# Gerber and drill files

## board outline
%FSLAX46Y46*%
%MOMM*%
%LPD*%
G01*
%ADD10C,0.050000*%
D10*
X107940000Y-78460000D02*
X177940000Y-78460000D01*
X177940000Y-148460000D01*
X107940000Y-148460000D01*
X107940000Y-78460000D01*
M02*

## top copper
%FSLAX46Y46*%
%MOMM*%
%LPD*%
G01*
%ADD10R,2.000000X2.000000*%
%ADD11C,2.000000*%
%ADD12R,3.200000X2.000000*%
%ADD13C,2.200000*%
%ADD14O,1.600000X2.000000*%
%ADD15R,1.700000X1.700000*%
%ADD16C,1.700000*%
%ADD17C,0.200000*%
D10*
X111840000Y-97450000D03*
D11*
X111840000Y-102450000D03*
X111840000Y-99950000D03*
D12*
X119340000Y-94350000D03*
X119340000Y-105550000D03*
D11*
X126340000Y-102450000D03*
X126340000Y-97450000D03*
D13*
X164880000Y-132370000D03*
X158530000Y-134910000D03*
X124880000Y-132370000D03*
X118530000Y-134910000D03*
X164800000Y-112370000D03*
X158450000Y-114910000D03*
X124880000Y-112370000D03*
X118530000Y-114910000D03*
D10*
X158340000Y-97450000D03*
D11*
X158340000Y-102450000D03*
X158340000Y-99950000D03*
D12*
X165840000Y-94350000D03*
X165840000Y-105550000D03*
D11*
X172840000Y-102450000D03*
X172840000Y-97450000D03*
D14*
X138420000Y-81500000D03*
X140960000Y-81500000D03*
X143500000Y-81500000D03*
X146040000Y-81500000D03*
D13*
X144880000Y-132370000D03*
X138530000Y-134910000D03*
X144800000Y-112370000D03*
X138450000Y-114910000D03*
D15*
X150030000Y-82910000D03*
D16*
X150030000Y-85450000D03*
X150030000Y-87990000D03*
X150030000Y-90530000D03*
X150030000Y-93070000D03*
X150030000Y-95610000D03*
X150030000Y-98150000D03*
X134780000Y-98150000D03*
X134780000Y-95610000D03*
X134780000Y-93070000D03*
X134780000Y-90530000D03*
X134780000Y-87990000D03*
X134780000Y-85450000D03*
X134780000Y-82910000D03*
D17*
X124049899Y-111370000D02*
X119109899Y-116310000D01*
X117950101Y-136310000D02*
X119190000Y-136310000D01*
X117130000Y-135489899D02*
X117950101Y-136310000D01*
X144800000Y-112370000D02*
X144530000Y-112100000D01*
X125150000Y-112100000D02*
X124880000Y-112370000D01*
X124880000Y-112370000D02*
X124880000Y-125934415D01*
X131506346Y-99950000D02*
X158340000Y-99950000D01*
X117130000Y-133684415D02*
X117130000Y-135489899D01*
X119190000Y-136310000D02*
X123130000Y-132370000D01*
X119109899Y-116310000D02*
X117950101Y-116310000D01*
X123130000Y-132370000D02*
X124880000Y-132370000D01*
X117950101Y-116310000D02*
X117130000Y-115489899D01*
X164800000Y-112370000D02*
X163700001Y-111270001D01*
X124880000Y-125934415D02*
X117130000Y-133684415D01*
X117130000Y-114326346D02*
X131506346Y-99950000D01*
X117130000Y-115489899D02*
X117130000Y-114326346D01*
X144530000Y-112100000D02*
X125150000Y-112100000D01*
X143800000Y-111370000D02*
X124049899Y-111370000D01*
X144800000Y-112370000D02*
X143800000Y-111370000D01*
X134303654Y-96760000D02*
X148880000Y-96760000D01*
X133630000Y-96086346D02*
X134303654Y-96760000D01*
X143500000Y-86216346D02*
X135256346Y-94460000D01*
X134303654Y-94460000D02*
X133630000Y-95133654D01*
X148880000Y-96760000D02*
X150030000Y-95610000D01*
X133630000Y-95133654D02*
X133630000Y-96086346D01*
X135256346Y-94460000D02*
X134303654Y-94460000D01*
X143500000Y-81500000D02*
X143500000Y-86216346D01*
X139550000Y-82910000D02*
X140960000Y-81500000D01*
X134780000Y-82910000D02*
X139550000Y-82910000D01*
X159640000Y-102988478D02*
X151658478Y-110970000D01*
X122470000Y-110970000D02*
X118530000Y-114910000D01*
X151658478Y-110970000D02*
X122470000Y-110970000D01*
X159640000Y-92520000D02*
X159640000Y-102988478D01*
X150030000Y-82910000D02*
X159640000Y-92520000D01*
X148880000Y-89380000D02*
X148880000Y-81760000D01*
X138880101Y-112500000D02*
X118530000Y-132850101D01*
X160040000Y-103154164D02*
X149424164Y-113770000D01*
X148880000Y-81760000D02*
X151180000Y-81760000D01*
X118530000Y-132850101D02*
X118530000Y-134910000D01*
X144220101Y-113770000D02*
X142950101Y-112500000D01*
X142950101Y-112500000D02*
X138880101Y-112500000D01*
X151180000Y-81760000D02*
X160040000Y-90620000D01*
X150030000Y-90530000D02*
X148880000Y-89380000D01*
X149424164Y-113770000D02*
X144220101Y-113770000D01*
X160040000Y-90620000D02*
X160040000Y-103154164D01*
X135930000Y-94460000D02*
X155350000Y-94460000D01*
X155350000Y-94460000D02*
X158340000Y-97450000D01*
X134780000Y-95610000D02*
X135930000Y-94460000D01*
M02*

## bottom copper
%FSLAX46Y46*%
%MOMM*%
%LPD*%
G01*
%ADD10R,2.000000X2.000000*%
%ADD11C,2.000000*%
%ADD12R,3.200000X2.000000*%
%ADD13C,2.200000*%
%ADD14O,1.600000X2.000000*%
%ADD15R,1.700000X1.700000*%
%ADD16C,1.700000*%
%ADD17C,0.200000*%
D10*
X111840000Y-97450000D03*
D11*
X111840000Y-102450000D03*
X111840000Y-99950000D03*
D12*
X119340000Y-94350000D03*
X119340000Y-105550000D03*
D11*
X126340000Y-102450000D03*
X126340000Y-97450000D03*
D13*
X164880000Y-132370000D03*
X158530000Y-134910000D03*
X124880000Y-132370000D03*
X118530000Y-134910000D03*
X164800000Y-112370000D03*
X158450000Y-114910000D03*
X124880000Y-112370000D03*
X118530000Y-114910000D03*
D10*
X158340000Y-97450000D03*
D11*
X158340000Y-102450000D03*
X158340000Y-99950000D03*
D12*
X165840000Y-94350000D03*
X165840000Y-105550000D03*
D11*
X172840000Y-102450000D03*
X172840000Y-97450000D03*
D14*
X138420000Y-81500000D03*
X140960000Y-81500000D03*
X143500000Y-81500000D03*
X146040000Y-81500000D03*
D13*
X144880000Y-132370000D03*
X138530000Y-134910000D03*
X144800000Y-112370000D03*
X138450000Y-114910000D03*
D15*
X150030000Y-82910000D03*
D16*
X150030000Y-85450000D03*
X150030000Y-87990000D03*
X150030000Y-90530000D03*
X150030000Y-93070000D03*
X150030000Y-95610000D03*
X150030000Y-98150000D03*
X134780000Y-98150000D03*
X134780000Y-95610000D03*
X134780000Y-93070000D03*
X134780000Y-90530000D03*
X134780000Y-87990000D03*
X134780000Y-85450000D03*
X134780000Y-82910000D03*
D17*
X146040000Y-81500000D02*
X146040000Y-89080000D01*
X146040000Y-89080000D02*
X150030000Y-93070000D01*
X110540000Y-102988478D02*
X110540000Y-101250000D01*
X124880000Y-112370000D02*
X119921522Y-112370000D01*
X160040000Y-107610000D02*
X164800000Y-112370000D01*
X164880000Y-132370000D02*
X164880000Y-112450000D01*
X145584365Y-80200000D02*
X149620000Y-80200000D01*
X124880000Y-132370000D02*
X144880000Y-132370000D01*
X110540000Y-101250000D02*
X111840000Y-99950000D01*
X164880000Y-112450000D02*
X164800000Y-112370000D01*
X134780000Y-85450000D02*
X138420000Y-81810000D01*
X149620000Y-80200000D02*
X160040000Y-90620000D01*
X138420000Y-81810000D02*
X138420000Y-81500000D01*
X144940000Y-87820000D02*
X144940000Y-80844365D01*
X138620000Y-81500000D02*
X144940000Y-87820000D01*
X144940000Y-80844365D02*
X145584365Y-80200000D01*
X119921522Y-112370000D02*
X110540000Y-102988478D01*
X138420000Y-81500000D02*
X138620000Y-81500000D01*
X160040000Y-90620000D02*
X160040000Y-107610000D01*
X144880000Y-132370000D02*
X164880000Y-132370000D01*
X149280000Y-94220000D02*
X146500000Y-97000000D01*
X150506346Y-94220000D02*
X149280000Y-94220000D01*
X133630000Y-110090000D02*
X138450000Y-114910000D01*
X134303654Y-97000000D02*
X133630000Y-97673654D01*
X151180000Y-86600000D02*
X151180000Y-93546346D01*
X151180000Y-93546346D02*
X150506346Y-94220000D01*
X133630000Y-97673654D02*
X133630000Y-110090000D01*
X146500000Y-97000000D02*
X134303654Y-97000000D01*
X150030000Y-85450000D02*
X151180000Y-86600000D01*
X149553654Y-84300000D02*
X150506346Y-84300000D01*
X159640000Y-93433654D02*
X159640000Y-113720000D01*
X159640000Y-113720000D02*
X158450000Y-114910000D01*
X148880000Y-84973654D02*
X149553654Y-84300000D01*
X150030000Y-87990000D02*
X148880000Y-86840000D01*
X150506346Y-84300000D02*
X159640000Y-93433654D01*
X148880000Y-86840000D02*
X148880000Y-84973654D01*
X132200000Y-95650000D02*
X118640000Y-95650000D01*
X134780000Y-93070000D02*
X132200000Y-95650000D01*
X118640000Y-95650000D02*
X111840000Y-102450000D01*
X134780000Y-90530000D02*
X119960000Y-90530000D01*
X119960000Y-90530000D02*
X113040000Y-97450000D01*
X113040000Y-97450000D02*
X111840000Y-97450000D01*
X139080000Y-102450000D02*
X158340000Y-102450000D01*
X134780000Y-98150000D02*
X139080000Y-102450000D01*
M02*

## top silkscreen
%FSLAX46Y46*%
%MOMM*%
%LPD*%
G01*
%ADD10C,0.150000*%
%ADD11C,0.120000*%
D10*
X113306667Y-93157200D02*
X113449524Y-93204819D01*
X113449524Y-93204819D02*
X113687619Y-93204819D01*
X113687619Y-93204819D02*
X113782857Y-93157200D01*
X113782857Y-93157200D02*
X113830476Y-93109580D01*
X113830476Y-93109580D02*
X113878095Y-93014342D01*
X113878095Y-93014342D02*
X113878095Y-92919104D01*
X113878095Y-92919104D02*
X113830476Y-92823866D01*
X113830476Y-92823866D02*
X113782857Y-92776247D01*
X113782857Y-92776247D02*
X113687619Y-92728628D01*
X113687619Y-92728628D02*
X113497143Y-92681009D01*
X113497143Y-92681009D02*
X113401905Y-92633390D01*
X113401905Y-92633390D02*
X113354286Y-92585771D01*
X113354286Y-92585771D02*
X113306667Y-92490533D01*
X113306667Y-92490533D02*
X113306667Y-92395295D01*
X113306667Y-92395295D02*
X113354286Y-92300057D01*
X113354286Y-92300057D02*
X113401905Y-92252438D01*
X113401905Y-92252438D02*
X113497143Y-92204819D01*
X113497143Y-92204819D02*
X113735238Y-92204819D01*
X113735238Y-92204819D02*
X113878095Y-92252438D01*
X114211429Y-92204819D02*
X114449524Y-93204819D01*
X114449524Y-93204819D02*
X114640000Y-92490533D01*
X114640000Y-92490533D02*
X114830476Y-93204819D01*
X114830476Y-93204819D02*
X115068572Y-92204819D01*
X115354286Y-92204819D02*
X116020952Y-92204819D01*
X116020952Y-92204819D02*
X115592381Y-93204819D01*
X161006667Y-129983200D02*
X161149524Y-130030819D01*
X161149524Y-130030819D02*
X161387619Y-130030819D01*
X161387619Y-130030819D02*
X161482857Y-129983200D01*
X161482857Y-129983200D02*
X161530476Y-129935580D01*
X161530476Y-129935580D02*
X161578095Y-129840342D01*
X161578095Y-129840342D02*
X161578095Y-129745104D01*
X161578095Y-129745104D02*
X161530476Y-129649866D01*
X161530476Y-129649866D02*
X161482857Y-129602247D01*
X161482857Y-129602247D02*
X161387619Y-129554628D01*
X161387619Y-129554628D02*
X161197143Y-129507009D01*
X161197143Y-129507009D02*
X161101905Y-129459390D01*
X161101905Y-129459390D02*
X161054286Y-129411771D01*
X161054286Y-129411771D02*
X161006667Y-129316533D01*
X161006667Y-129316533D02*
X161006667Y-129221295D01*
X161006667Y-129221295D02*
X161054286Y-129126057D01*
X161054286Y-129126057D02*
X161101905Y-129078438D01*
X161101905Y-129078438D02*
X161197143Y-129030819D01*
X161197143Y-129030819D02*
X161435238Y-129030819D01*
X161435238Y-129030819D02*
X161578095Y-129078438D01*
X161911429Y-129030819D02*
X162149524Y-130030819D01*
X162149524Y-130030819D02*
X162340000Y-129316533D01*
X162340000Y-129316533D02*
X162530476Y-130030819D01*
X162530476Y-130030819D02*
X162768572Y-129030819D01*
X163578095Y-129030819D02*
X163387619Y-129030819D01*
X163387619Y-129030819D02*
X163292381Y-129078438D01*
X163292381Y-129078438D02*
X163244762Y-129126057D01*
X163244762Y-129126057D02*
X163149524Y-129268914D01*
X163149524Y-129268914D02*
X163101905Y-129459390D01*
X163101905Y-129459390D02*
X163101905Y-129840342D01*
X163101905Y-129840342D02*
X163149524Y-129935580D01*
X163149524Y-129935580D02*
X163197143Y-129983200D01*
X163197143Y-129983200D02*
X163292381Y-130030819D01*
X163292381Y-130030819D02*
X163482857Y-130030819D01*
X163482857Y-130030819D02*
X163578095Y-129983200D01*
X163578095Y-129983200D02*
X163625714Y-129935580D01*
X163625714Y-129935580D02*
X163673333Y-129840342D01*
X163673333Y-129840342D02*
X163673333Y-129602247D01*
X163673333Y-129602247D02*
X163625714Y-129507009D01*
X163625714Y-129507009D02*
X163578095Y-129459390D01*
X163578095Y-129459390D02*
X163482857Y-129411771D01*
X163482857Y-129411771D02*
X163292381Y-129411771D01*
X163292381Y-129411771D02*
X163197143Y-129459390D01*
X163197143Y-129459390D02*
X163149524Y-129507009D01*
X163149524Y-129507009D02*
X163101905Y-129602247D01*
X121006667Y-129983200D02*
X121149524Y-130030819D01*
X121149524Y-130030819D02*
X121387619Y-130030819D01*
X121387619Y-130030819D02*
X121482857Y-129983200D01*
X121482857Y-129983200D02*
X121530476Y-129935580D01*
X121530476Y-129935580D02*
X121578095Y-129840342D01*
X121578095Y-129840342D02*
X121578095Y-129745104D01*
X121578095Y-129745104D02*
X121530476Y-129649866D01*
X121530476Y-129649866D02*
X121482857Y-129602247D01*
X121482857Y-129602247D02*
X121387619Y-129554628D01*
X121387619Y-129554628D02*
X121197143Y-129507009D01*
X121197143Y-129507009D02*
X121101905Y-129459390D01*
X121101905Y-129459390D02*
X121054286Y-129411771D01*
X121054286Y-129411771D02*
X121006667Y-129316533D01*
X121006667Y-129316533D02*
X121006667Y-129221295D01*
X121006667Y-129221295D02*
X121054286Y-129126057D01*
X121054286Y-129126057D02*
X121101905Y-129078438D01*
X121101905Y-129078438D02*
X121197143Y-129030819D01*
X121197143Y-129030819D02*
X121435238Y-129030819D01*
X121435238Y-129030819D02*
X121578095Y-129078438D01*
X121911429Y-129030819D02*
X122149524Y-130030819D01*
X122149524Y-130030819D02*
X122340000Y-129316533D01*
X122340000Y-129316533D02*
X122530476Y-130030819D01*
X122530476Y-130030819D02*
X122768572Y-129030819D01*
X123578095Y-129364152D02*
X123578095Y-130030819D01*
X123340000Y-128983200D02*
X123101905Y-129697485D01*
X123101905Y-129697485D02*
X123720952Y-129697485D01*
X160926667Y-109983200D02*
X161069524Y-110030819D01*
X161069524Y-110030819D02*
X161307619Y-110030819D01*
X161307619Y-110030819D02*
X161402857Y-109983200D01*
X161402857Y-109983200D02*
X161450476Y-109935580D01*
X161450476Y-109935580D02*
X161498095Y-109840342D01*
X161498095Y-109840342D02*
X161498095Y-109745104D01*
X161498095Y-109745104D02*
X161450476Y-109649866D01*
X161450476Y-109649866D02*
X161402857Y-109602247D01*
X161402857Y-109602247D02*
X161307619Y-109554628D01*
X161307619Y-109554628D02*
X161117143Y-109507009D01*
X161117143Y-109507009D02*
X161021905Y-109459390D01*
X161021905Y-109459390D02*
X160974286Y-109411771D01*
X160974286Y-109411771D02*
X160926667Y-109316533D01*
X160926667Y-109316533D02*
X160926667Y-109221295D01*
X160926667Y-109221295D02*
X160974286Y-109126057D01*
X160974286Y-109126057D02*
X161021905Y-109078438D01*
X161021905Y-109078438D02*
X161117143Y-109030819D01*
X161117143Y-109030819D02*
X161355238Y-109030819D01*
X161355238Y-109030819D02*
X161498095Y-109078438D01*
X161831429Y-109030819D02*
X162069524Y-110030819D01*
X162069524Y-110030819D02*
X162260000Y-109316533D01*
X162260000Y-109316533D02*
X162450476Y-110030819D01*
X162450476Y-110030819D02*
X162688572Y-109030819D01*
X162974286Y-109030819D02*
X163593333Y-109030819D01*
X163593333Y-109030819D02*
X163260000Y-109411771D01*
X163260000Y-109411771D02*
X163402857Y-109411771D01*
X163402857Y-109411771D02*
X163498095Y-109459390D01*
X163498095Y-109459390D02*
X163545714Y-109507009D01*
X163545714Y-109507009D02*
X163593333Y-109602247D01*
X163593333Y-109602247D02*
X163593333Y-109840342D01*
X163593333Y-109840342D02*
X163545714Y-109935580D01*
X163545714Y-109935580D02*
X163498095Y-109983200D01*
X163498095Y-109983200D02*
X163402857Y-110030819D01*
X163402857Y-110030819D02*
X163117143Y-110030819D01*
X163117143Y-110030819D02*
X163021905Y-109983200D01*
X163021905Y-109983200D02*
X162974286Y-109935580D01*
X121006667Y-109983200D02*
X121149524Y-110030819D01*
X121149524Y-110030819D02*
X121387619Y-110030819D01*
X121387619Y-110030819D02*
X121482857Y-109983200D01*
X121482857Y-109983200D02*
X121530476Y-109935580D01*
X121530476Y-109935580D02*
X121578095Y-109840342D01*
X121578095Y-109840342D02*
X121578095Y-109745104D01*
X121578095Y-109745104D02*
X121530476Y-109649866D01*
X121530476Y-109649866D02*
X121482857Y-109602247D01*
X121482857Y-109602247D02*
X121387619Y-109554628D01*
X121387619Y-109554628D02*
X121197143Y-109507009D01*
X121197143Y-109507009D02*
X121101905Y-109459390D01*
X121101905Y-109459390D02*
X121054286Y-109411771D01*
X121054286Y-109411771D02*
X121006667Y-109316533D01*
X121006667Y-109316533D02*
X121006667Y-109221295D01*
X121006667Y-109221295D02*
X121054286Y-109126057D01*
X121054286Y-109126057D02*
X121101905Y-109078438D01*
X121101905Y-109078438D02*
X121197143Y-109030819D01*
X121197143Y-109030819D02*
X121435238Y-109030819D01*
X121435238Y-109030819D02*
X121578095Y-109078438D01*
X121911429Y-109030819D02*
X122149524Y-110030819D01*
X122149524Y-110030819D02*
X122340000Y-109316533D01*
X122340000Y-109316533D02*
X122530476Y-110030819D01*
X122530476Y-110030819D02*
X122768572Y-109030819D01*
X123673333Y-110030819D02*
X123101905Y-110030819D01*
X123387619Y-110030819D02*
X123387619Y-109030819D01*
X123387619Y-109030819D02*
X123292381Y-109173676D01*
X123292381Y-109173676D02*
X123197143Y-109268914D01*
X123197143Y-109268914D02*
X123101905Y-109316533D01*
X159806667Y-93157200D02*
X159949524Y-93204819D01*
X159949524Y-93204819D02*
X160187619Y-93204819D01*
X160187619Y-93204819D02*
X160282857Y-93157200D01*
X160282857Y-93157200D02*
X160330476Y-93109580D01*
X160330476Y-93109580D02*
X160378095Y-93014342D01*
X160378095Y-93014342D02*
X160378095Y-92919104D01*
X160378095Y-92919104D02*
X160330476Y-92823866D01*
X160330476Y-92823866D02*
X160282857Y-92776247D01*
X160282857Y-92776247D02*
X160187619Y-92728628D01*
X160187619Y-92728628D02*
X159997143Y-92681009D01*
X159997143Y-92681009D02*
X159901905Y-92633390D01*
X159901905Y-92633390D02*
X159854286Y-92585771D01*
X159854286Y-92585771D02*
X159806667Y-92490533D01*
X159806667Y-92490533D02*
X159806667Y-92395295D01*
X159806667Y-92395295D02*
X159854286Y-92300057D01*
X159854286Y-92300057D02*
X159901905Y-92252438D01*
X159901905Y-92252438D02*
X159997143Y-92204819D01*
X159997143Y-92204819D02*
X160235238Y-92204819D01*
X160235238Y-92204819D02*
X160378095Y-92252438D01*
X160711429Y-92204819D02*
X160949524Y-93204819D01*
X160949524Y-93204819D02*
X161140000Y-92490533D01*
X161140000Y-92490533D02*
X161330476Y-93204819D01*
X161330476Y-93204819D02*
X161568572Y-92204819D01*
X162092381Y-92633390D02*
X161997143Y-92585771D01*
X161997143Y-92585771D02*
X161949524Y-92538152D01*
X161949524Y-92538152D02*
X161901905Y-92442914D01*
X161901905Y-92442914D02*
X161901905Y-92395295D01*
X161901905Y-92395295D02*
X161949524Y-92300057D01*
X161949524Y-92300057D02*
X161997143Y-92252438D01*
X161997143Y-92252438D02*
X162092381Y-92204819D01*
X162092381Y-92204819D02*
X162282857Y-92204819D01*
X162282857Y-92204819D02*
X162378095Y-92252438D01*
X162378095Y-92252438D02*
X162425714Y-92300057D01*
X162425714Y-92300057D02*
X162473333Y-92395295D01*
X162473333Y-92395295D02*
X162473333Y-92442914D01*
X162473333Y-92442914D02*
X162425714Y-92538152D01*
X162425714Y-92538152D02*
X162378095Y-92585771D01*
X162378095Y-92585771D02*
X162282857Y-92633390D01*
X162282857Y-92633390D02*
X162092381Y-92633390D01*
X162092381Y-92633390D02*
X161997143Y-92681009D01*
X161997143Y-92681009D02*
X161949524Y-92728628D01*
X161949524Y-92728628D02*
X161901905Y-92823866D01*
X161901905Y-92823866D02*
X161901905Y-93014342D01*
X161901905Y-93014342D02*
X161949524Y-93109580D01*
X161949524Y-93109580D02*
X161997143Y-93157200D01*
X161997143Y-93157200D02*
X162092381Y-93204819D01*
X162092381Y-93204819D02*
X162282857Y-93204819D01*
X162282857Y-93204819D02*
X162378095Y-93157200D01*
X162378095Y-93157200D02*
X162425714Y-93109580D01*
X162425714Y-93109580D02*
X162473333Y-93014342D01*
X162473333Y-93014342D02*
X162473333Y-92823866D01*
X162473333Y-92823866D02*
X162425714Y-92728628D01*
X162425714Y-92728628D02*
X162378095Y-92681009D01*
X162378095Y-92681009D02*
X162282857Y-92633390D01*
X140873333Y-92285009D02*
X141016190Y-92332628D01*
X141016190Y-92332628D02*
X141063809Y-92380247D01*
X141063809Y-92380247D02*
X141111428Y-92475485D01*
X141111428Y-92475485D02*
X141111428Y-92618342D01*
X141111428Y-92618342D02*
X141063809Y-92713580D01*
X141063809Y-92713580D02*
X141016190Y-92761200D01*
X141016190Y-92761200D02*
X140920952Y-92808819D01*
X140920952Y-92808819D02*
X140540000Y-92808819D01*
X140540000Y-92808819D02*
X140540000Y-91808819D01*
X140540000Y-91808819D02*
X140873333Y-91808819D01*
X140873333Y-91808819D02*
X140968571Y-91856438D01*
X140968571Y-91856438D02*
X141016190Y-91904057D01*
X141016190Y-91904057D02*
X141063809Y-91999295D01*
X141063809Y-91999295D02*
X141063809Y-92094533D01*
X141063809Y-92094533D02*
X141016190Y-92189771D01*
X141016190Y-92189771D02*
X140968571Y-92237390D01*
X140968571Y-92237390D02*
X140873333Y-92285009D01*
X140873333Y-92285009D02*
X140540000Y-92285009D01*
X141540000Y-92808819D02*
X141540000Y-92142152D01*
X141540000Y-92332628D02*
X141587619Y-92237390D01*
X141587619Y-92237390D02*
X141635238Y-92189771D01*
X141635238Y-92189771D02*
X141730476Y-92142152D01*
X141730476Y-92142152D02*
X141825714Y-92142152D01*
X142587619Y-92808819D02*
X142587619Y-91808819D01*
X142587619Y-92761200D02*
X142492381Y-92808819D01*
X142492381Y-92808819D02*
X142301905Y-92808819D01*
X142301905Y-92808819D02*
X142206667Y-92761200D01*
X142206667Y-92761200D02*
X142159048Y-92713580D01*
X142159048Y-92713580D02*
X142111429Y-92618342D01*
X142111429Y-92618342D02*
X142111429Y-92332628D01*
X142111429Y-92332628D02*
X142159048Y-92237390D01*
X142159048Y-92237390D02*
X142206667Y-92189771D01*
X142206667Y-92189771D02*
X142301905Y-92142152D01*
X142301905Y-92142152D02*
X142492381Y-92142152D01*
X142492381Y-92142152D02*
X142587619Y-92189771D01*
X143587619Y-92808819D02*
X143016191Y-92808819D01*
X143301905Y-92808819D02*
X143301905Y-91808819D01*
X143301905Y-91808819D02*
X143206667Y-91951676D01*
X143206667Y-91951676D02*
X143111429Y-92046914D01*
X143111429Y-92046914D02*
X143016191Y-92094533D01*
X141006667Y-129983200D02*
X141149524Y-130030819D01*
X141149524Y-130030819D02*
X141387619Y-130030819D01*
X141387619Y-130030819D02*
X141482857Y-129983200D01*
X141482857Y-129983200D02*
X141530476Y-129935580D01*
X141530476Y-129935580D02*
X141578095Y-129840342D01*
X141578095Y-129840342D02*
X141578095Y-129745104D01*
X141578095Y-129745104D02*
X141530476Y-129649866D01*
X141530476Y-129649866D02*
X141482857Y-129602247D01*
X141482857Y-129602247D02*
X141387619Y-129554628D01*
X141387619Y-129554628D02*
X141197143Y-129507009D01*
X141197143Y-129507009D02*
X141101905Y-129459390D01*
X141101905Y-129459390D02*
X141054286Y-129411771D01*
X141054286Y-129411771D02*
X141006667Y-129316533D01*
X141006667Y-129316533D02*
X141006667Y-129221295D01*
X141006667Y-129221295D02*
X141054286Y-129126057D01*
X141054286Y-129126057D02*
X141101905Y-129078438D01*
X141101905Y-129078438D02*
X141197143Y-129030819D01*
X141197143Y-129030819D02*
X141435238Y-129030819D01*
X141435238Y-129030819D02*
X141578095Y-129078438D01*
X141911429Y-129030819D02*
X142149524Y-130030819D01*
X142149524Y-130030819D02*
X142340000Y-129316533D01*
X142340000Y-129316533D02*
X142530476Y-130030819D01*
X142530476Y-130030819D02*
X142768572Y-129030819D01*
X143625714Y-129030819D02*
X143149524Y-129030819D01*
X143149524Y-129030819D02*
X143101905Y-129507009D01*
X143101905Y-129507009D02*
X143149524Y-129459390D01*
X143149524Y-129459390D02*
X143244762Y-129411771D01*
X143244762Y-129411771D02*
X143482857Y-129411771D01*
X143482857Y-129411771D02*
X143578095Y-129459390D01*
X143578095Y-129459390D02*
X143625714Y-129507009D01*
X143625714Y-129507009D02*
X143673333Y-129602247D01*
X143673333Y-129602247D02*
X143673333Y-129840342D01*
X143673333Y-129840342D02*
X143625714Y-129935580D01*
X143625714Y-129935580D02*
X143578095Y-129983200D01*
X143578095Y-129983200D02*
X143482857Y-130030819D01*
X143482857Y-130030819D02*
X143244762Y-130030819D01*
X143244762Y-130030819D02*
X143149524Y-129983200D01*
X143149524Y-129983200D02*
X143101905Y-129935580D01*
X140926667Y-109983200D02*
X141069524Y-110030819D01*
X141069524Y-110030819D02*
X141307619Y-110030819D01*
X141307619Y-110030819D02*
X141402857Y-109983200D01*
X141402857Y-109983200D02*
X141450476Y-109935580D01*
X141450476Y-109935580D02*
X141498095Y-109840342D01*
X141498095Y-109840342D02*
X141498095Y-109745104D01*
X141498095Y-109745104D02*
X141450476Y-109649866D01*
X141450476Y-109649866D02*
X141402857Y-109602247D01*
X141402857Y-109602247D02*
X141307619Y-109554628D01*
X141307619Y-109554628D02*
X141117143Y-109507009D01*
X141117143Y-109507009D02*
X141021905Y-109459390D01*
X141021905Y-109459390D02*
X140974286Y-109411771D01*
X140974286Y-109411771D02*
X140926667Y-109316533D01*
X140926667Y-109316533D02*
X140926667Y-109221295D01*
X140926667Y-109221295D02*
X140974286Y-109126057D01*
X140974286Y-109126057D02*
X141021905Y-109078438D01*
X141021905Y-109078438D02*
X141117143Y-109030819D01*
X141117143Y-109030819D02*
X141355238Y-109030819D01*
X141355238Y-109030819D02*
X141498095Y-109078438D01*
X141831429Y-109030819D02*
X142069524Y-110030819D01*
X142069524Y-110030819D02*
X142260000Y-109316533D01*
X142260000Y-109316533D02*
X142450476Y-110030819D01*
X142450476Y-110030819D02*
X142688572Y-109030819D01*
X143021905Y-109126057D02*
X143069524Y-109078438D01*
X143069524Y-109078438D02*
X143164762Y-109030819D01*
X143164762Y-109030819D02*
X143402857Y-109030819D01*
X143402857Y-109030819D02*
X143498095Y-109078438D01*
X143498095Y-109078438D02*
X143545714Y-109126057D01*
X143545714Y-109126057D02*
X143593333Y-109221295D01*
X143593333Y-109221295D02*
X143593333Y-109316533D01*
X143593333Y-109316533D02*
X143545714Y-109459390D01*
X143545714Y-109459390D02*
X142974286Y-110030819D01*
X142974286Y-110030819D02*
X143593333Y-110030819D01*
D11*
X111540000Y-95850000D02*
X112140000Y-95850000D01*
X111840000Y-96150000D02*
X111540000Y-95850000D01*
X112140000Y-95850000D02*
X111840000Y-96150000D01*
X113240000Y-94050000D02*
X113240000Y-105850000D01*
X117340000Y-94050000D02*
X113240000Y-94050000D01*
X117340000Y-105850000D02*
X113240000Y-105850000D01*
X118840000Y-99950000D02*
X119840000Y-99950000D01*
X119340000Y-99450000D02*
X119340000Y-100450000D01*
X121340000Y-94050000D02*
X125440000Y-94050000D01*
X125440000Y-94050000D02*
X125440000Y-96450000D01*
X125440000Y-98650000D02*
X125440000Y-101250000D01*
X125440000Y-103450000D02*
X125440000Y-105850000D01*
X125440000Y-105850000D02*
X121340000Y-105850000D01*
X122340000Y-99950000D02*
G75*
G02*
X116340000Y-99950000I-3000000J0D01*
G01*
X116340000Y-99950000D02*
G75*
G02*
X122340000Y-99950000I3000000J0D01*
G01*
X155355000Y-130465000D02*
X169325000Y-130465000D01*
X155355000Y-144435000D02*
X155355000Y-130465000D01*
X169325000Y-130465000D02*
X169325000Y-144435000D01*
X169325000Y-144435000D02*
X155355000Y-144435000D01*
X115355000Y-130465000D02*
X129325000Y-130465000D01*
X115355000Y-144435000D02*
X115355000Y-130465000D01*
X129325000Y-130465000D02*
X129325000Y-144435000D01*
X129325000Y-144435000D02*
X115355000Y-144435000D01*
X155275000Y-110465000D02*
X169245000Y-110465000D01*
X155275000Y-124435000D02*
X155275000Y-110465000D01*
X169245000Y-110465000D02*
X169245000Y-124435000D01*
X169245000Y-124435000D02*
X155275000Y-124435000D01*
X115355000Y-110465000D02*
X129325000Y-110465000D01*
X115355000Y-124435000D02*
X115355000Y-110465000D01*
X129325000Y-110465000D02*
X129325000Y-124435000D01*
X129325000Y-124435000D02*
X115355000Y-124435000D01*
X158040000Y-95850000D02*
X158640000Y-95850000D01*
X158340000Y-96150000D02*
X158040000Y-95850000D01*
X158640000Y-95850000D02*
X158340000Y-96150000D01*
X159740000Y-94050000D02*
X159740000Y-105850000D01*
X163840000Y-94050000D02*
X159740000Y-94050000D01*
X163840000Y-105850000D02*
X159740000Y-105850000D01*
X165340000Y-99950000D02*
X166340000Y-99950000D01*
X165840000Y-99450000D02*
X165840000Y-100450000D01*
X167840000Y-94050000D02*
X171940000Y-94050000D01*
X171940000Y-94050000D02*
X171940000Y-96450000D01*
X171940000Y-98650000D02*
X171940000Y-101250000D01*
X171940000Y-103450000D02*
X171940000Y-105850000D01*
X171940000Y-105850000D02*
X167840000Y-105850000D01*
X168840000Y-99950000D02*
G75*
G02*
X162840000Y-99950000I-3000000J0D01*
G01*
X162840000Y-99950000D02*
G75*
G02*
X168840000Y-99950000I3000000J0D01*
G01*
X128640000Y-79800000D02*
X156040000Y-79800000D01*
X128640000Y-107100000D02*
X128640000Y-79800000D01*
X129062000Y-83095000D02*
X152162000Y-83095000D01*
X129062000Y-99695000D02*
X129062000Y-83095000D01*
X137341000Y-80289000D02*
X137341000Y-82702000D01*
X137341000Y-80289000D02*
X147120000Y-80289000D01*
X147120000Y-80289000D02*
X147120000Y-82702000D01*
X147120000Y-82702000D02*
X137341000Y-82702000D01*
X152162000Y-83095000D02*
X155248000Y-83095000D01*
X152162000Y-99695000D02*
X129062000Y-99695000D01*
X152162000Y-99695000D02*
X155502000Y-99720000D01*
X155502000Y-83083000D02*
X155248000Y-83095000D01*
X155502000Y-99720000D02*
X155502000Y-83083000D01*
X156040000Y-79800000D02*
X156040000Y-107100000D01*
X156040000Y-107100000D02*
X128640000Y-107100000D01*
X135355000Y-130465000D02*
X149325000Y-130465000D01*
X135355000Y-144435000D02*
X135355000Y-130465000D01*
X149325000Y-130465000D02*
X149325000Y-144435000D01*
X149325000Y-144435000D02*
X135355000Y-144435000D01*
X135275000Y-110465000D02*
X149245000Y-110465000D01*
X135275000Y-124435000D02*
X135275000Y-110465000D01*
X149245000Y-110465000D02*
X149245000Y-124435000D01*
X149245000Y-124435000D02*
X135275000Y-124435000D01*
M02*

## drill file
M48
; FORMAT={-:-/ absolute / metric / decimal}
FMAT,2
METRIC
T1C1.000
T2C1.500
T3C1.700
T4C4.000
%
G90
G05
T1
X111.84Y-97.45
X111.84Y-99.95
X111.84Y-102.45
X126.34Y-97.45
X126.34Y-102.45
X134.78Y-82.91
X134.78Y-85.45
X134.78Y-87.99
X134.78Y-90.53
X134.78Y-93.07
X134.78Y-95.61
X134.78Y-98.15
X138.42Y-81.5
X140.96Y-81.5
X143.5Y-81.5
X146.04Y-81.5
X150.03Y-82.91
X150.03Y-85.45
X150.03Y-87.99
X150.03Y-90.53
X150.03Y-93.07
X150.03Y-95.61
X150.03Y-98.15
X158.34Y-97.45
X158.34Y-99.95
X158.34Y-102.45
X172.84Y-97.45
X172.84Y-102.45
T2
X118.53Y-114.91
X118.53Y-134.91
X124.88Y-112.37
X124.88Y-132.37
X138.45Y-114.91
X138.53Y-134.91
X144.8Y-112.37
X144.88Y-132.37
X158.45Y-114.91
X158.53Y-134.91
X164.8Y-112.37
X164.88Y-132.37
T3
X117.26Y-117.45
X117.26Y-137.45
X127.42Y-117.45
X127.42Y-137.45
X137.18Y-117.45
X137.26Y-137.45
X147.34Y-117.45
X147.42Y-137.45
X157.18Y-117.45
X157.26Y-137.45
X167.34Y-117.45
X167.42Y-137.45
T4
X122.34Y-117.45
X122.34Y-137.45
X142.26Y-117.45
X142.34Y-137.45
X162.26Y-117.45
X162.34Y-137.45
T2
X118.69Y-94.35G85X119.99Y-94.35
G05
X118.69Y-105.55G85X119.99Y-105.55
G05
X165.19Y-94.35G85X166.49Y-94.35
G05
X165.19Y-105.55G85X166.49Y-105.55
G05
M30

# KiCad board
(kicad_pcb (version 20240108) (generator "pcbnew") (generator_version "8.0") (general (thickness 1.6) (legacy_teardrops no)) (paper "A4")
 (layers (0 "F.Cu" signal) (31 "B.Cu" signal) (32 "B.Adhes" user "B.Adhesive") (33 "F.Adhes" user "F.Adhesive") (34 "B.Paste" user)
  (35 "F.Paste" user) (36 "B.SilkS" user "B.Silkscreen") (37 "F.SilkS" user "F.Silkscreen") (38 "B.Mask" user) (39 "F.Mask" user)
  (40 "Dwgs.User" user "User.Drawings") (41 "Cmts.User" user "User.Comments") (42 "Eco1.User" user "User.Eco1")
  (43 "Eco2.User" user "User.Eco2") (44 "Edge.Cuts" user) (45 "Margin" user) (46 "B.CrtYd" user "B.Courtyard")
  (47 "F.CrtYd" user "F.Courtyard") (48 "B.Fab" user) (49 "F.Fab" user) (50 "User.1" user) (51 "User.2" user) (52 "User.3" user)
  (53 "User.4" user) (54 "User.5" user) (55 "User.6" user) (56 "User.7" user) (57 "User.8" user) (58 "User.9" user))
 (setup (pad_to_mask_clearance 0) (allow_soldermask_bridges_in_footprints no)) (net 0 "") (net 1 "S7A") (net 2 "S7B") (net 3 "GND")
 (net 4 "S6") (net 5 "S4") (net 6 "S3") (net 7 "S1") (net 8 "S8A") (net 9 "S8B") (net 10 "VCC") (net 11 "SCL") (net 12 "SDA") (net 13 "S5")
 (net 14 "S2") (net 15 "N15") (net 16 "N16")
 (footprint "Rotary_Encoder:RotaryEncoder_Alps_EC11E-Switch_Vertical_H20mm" (layer "F.Cu") (at 111.84 97.45)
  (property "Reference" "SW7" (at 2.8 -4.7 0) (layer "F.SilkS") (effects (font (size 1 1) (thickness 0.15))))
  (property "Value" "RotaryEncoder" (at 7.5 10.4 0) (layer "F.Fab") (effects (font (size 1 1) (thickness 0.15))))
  (fp_line (start -0.3 -1.6) (end 0.3 -1.6) (stroke (width 0.12) (type solid)) (layer "F.SilkS"))
  (fp_line (start 0 -1.3) (end -0.3 -1.6) (stroke (width 0.12) (type solid)) (layer "F.SilkS"))
  (fp_line (start 0.3 -1.6) (end 0 -1.3) (stroke (width 0.12) (type solid)) (layer "F.SilkS"))
  (fp_line (start 1.4 -3.4) (end 1.4 8.4) (stroke (width 0.12) (type solid)) (layer "F.SilkS"))
  (fp_line (start 5.5 -3.4) (end 1.4 -3.4) (stroke (width 0.12) (type solid)) (layer "F.SilkS"))
  (fp_line (start 5.5 8.4) (end 1.4 8.4) (stroke (width 0.12) (type solid)) (layer "F.SilkS"))
  (fp_line (start 7 2.5) (end 8 2.5) (stroke (width 0.12) (type solid)) (layer "F.SilkS"))
  (fp_line (start 7.5 2) (end 7.5 3) (stroke (width 0.12) (type solid)) (layer "F.SilkS"))
  (fp_line (start 9.5 -3.4) (end 13.6 -3.4) (stroke (width 0.12) (type solid)) (layer "F.SilkS"))
  (fp_line (start 13.6 -3.4) (end 13.6 -1) (stroke (width 0.12) (type solid)) (layer "F.SilkS"))
  (fp_line (start 13.6 1.2) (end 13.6 3.8) (stroke (width 0.12) (type solid)) (layer "F.SilkS"))
  (fp_line (start 13.6 6) (end 13.6 8.4) (stroke (width 0.12) (type solid)) (layer "F.SilkS"))
  (fp_line (start 13.6 8.4) (end 9.5 8.4) (stroke (width 0.12) (type solid)) (layer "F.SilkS"))
  (fp_circle (center 7.5 2.5) (end 10.5 2.5) (stroke (width 0.12) (type solid)) (fill none) (layer "F.SilkS"))
  (pad "A" thru_hole rect (at 0 0) (size 2 2) (drill 1) (layers "*.Cu" "*.Mask") (remove_unused_layers no) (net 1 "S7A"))
  (pad "B" thru_hole circle (at 0 5) (size 2 2) (drill 1) (layers "*.Cu" "*.Mask") (remove_unused_layers no) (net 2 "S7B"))
  (pad "C" thru_hole circle (at 0 2.5) (size 2 2) (drill 1) (layers "*.Cu" "*.Mask") (remove_unused_layers no) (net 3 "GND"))
  (pad "MP" thru_hole rect (at 7.5 -3.1) (size 3.2 2) (drill oval 2.8 1.5) (layers "*.Cu" "*.Mask") (remove_unused_layers no))
  (pad "MP" thru_hole rect (at 7.5 8.1) (size 3.2 2) (drill oval 2.8 1.5) (layers "*.Cu" "*.Mask") (remove_unused_layers no))
  (pad "S1" thru_hole circle (at 14.5 5) (size 2 2) (drill 1) (layers "*.Cu" "*.Mask") (remove_unused_layers no))
  (pad "S2" thru_hole circle (at 14.5 0) (size 2 2) (drill 1) (layers "*.Cu" "*.Mask") (remove_unused_layers no)))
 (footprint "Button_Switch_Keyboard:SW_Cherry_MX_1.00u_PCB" (layer "F.Cu") (at 164.88 132.37)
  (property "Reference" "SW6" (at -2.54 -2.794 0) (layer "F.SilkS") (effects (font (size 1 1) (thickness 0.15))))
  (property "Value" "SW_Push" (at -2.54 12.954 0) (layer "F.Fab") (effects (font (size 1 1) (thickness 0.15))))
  (fp_line (start -9.525 -1.905) (end 4.445 -1.905) (stroke (width 0.12) (type solid)) (layer "F.SilkS"))
  (fp_line (start -9.525 12.065) (end -9.525 -1.905) (stroke (width 0.12) (type solid)) (layer "F.SilkS"))
  (fp_line (start 4.445 -1.905) (end 4.445 12.065) (stroke (width 0.12) (type solid)) (layer "F.SilkS"))
  (fp_line (start 4.445 12.065) (end -9.525 12.065) (stroke (width 0.12) (type solid)) (layer "F.SilkS"))
  (pad "" np_thru_hole circle (at -7.62 5.08) (size 1.7 1.7) (drill 1.7) (layers "*.Cu" "*.Mask"))
  (pad "" np_thru_hole circle (at -2.54 5.08) (size 4 4) (drill 4) (layers "*.Cu" "*.Mask"))
  (pad "" np_thru_hole circle (at 2.54 5.08) (size 1.7 1.7) (drill 1.7) (layers "*.Cu" "*.Mask"))
  (pad "1" thru_hole circle (at 0 0) (size 2.2 2.2) (drill 1.5) (layers "*.Cu" "*.Mask") (remove_unused_layers no) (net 3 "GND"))
  (pad "2" thru_hole circle (at -6.35 2.54) (size 2.2 2.2) (drill 1.5) (layers "*.Cu" "*.Mask") (remove_unused_layers no) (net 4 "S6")))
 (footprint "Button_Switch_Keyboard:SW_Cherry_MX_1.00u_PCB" (layer "F.Cu") (at 124.88 132.37)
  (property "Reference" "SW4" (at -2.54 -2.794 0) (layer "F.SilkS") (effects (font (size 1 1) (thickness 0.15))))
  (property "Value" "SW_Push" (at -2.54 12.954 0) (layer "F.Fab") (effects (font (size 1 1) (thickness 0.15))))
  (fp_line (start -9.525 -1.905) (end 4.445 -1.905) (stroke (width 0.12) (type solid)) (layer "F.SilkS"))
  (fp_line (start -9.525 12.065) (end -9.525 -1.905) (stroke (width 0.12) (type solid)) (layer "F.SilkS"))
  (fp_line (start 4.445 -1.905) (end 4.445 12.065) (stroke (width 0.12) (type solid)) (layer "F.SilkS"))
  (fp_line (start 4.445 12.065) (end -9.525 12.065) (stroke (width 0.12) (type solid)) (layer "F.SilkS"))
  (pad "" np_thru_hole circle (at -7.62 5.08) (size 1.7 1.7) (drill 1.7) (layers "*.Cu" "*.Mask"))
  (pad "" np_thru_hole circle (at -2.54 5.08) (size 4 4) (drill 4) (layers "*.Cu" "*.Mask"))
  (pad "" np_thru_hole circle (at 2.54 5.08) (size 1.7 1.7) (drill 1.7) (layers "*.Cu" "*.Mask"))
  (pad "1" thru_hole circle (at 0 0) (size 2.2 2.2) (drill 1.5) (layers "*.Cu" "*.Mask") (remove_unused_layers no) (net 3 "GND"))
  (pad "2" thru_hole circle (at -6.35 2.54) (size 2.2 2.2) (drill 1.5) (layers "*.Cu" "*.Mask") (remove_unused_layers no) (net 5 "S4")))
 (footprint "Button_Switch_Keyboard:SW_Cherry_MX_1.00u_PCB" (layer "F.Cu") (at 164.8 112.37)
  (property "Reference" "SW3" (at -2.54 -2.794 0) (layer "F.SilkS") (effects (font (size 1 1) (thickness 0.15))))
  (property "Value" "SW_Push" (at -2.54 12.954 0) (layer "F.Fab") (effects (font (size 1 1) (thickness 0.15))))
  (fp_line (start -9.525 -1.905) (end 4.445 -1.905) (stroke (width 0.12) (type solid)) (layer "F.SilkS"))
  (fp_line (start -9.525 12.065) (end -9.525 -1.905) (stroke (width 0.12) (type solid)) (layer "F.SilkS"))
  (fp_line (start 4.445 -1.905) (end 4.445 12.065) (stroke (width 0.12) (type solid)) (layer "F.SilkS"))
  (fp_line (start 4.445 12.065) (end -9.525 12.065) (stroke (width 0.12) (type solid)) (layer "F.SilkS"))
  (pad "" np_thru_hole circle (at -7.62 5.08) (size 1.7 1.7) (drill 1.7) (layers "*.Cu" "*.Mask"))
  (pad "" np_thru_hole circle (at -2.54 5.08) (size 4 4) (drill 4) (layers "*.Cu" "*.Mask"))
  (pad "" np_thru_hole circle (at 2.54 5.08) (size 1.7 1.7) (drill 1.7) (layers "*.Cu" "*.Mask"))
  (pad "1" thru_hole circle (at 0 0) (size 2.2 2.2) (drill 1.5) (layers "*.Cu" "*.Mask") (remove_unused_layers no) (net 3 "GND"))
  (pad "2" thru_hole circle (at -6.35 2.54) (size 2.2 2.2) (drill 1.5) (layers "*.Cu" "*.Mask") (remove_unused_layers no) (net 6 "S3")))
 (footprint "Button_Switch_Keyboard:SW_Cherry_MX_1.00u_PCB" (layer "F.Cu") (at 124.88 112.37)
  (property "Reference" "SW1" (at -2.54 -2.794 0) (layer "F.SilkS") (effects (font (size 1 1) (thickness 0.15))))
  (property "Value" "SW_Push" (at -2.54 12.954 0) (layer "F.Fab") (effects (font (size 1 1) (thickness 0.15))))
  (fp_line (start -9.525 -1.905) (end 4.445 -1.905) (stroke (width 0.12) (type solid)) (layer "F.SilkS"))
  (fp_line (start -9.525 12.065) (end -9.525 -1.905) (stroke (width 0.12) (type solid)) (layer "F.SilkS"))
  (fp_line (start 4.445 -1.905) (end 4.445 12.065) (stroke (width 0.12) (type solid)) (layer "F.SilkS"))
  (fp_line (start 4.445 12.065) (end -9.525 12.065) (stroke (width 0.12) (type solid)) (layer "F.SilkS"))
  (pad "" np_thru_hole circle (at -7.62 5.08) (size 1.7 1.7) (drill 1.7) (layers "*.Cu" "*.Mask"))
  (pad "" np_thru_hole circle (at -2.54 5.08) (size 4 4) (drill 4) (layers "*.Cu" "*.Mask"))
  (pad "" np_thru_hole circle (at 2.54 5.08) (size 1.7 1.7) (drill 1.7) (layers "*.Cu" "*.Mask"))
  (pad "1" thru_hole circle (at 0 0) (size 2.2 2.2) (drill 1.5) (layers "*.Cu" "*.Mask") (remove_unused_layers no) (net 3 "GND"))
  (pad "2" thru_hole circle (at -6.35 2.54) (size 2.2 2.2) (drill 1.5) (layers "*.Cu" "*.Mask") (remove_unused_layers no) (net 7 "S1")))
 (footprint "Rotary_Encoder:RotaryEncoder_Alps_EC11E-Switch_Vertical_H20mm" (layer "F.Cu") (at 158.34 97.45)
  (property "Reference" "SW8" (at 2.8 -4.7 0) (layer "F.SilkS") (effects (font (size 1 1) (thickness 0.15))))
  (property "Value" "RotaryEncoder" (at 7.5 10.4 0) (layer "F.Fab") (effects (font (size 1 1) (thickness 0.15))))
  (fp_line (start -0.3 -1.6) (end 0.3 -1.6) (stroke (width 0.12) (type solid)) (layer "F.SilkS"))
  (fp_line (start 0 -1.3) (end -0.3 -1.6) (stroke (width 0.12) (type solid)) (layer "F.SilkS"))
  (fp_line (start 0.3 -1.6) (end 0 -1.3) (stroke (width 0.12) (type solid)) (layer "F.SilkS"))
  (fp_line (start 1.4 -3.4) (end 1.4 8.4) (stroke (width 0.12) (type solid)) (layer "F.SilkS"))
  (fp_line (start 5.5 -3.4) (end 1.4 -3.4) (stroke (width 0.12) (type solid)) (layer "F.SilkS"))
  (fp_line (start 5.5 8.4) (end 1.4 8.4) (stroke (width 0.12) (type solid)) (layer "F.SilkS"))
  (fp_line (start 7 2.5) (end 8 2.5) (stroke (width 0.12) (type solid)) (layer "F.SilkS"))
  (fp_line (start 7.5 2) (end 7.5 3) (stroke (width 0.12) (type solid)) (layer "F.SilkS"))
  (fp_line (start 9.5 -3.4) (end 13.6 -3.4) (stroke (width 0.12) (type solid)) (layer "F.SilkS"))
  (fp_line (start 13.6 -3.4) (end 13.6 -1) (stroke (width 0.12) (type solid)) (layer "F.SilkS"))
  (fp_line (start 13.6 1.2) (end 13.6 3.8) (stroke (width 0.12) (type solid)) (layer "F.SilkS"))
  (fp_line (start 13.6 6) (end 13.6 8.4) (stroke (width 0.12) (type solid)) (layer "F.SilkS"))
  (fp_line (start 13.6 8.4) (end 9.5 8.4) (stroke (width 0.12) (type solid)) (layer "F.SilkS"))
  (fp_circle (center 7.5 2.5) (end 10.5 2.5) (stroke (width 0.12) (type solid)) (fill none) (layer "F.SilkS"))
  (pad "A" thru_hole rect (at 0 0) (size 2 2) (drill 1) (layers "*.Cu" "*.Mask") (remove_unused_layers no) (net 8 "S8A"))
  (pad "B" thru_hole circle (at 0 5) (size 2 2) (drill 1) (layers "*.Cu" "*.Mask") (remove_unused_layers no) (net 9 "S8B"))
  (pad "C" thru_hole circle (at 0 2.5) (size 2 2) (drill 1) (layers "*.Cu" "*.Mask") (remove_unused_layers no) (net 3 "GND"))
  (pad "MP" thru_hole rect (at 7.5 -3.1) (size 3.2 2) (drill oval 2.8 1.5) (layers "*.Cu" "*.Mask") (remove_unused_layers no))
  (pad "MP" thru_hole rect (at 7.5 8.1) (size 3.2 2) (drill oval 2.8 1.5) (layers "*.Cu" "*.Mask") (remove_unused_layers no))
  (pad "S1" thru_hole circle (at 14.5 5) (size 2 2) (drill 1) (layers "*.Cu" "*.Mask") (remove_unused_layers no))
  (pad "S2" thru_hole circle (at 14.5 0) (size 2 2) (drill 1) (layers "*.Cu" "*.Mask") (remove_unused_layers no)))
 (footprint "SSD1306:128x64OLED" (layer "F.Cu") (at 142.04 92.1)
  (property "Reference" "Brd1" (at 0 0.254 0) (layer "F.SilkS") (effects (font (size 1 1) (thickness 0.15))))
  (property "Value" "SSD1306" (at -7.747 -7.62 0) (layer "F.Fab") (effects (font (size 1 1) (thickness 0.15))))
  (fp_line (start -13.4 -12.3) (end 14 -12.3) (stroke (width 0.12) (type solid)) (layer "F.SilkS"))
  (fp_line (start -13.4 15) (end -13.4 -12.3) (stroke (width 0.12) (type solid)) (layer "F.SilkS"))
  (fp_line (start -12.978 -9.005) (end 10.122 -9.005) (stroke (width 0.12) (type solid)) (layer "F.SilkS"))
  (fp_line (start -12.978 7.595) (end -12.978 -9.005) (stroke (width 0.12) (type solid)) (layer "F.SilkS"))
  (fp_line (start -4.699 -11.811) (end -4.699 -9.398) (stroke (width 0.12) (type solid)) (layer "F.SilkS"))
  (fp_line (start -4.699 -11.811) (end 5.08 -11.811) (stroke (width 0.12) (type solid)) (layer "F.SilkS"))
  (fp_line (start 5.08 -11.811) (end 5.08 -9.398) (stroke (width 0.12) (type solid)) (layer "F.SilkS"))
  (fp_line (start 5.08 -9.398) (end -4.699 -9.398) (stroke (width 0.12) (type solid)) (layer "F.SilkS"))
  (fp_line (start 10.122 -9.005) (end 13.208 -9.005) (stroke (width 0.12) (type solid)) (layer "F.SilkS"))
  (fp_line (start 10.122 7.595) (end -12.978 7.595) (stroke (width 0.12) (type solid)) (layer "F.SilkS"))
  (fp_line (start 10.122 7.595) (end 13.462 7.62) (stroke (width 0.12) (type solid)) (layer "F.SilkS"))
  (fp_line (start 13.462 -9.017) (end 13.208 -9.005) (stroke (width 0.12) (type solid)) (layer "F.SilkS"))
  (fp_line (start 13.462 7.62) (end 13.462 -9.017) (stroke (width 0.12) (type solid)) (layer "F.SilkS"))
  (fp_line (start 14 -12.3) (end 14 15) (stroke (width 0.12) (type solid)) (layer "F.SilkS"))
  (fp_line (start 14 15) (end -13.4 15) (stroke (width 0.12) (type solid)) (layer "F.SilkS"))
  (pad "1" thru_hole oval (at -3.62 -10.6 90) (size 2 1.6) (drill 1) (layers "*.Cu" "*.Mask") (remove_unused_layers no) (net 3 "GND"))
  (pad "2" thru_hole oval (at -1.08 -10.6 90) (size 2 1.6) (drill 1) (layers "*.Cu" "*.Mask") (remove_unused_layers no) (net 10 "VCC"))
  (pad "3" thru_hole oval (at 1.46 -10.6 90) (size 2 1.6) (drill 1) (layers "*.Cu" "*.Mask") (remove_unused_layers no) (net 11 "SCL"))
  (pad "4" thru_hole oval (at 4 -10.6 90) (size 2 1.6) (drill 1) (layers "*.Cu" "*.Mask") (remove_unused_layers no) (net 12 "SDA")))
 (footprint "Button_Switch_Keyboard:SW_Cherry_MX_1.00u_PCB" (layer "F.Cu") (at 144.88 132.37)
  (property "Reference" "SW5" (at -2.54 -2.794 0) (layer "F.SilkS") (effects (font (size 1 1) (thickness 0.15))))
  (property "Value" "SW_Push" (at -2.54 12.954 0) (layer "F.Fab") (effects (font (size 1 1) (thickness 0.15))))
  (fp_line (start -9.525 -1.905) (end 4.445 -1.905) (stroke (width 0.12) (type solid)) (layer "F.SilkS"))
  (fp_line (start -9.525 12.065) (end -9.525 -1.905) (stroke (width 0.12) (type solid)) (layer "F.SilkS"))
  (fp_line (start 4.445 -1.905) (end 4.445 12.065) (stroke (width 0.12) (type solid)) (layer "F.SilkS"))
  (fp_line (start 4.445 12.065) (end -9.525 12.065) (stroke (width 0.12) (type solid)) (layer "F.SilkS"))
  (pad "" np_thru_hole circle (at -7.62 5.08) (size 1.7 1.7) (drill 1.7) (layers "*.Cu" "*.Mask"))
  (pad "" np_thru_hole circle (at -2.54 5.08) (size 4 4) (drill 4) (layers "*.Cu" "*.Mask"))
  (pad "" np_thru_hole circle (at 2.54 5.08) (size 1.7 1.7) (drill 1.7) (layers "*.Cu" "*.Mask"))
  (pad "1" thru_hole circle (at 0 0) (size 2.2 2.2) (drill 1.5) (layers "*.Cu" "*.Mask") (remove_unused_layers no) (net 3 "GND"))
  (pad "2" thru_hole circle (at -6.35 2.54) (size 2.2 2.2) (drill 1.5) (layers "*.Cu" "*.Mask") (remove_unused_layers no) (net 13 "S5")))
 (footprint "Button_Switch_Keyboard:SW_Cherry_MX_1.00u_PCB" (layer "F.Cu") (at 144.8 112.37)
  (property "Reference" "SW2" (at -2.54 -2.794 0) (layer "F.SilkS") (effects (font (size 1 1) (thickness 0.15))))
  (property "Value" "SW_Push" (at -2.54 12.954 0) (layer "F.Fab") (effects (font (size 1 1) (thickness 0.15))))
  (fp_line (start -9.525 -1.905) (end 4.445 -1.905) (stroke (width 0.12) (type solid)) (layer "F.SilkS"))
  (fp_line (start -9.525 12.065) (end -9.525 -1.905) (stroke (width 0.12) (type solid)) (layer "F.SilkS"))
  (fp_line (start 4.445 -1.905) (end 4.445 12.065) (stroke (width 0.12) (type solid)) (layer "F.SilkS"))
  (fp_line (start 4.445 12.065) (end -9.525 12.065) (stroke (width 0.12) (type solid)) (layer "F.SilkS"))
  (pad "" np_thru_hole circle (at -7.62 5.08) (size 1.7 1.7) (drill 1.7) (layers "*.Cu" "*.Mask"))
  (pad "" np_thru_hole circle (at -2.54 5.08) (size 4 4) (drill 4) (layers "*.Cu" "*.Mask"))
  (pad "" np_thru_hole circle (at 2.54 5.08) (size 1.7 1.7) (drill 1.7) (layers "*.Cu" "*.Mask"))
  (pad "1" thru_hole circle (at 0 0) (size 2.2 2.2) (drill 1.5) (layers "*.Cu" "*.Mask") (remove_unused_layers no) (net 3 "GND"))
  (pad "2" thru_hole circle (at -6.35 2.54) (size 2.2 2.2) (drill 1.5) (layers "*.Cu" "*.Mask") (remove_unused_layers no) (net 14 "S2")))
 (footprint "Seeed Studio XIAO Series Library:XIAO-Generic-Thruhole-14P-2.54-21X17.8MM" (layer "B.Cu") (at 142.405 90.53 180)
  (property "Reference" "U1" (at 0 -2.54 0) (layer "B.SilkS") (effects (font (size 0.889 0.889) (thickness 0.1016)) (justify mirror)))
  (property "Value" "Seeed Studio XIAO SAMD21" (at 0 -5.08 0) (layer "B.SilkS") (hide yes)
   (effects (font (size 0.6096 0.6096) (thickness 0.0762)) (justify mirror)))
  (pad "1" thru_hole rect (at -7.625 7.62 180) (size 1.7 1.7) (drill 1) (layers "*.Cu" "*.Mask") (remove_unused_layers no) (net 7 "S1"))
  (pad "2" thru_hole circle (at -7.625 5.08 180) (size 1.7 1.7) (drill 1) (layers "*.Cu" "*.Mask") (remove_unused_layers no) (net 14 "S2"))
  (pad "3" thru_hole circle (at -7.625 2.54 180) (size 1.7 1.7) (drill 1) (layers "*.Cu" "*.Mask") (remove_unused_layers no) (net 6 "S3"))
  (pad "4" thru_hole circle (at -7.625 0 180) (size 1.7 1.7) (drill 1) (layers "*.Cu" "*.Mask") (remove_unused_layers no) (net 5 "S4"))
  (pad "5" thru_hole circle (at -7.625 -2.54 180) (size 1.7 1.7) (drill 1) (layers "*.Cu" "*.Mask") (remove_unused_layers no) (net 12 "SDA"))
  (pad "6" thru_hole circle (at -7.625 -5.08) (size 1.7 1.7) (drill 1) (layers "*.Cu" "*.Mask") (remove_unused_layers no) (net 11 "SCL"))
  (pad "7" thru_hole circle (at -7.625 -7.62 180) (size 1.7 1.7) (drill 1) (layers "*.Cu" "*.Mask") (remove_unused_layers no) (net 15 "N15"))
  (pad "8" thru_hole circle (at 7.625 -7.62 180) (size 1.7 1.7) (drill 1) (layers "*.Cu" "*.Mask") (remove_unused_layers no) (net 9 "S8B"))
  (pad "9" thru_hole circle (at 7.625 -5.08 180) (size 1.7 1.7) (drill 1) (layers "*.Cu" "*.Mask") (remove_unused_layers no) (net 8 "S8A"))
  (pad "10" thru_hole circle (at 7.625 -2.54 180) (size 1.7 1.7) (drill 1) (layers "*.Cu" "*.Mask") (remove_unused_layers no) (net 2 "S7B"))
  (pad "11" thru_hole circle (at 7.625 0 180) (size 1.7 1.7) (drill 1) (layers "*.Cu" "*.Mask") (remove_unused_layers no) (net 1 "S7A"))
  (pad "12" thru_hole circle (at 7.625 2.54 180) (size 1.7 1.7) (drill 1) (layers "*.Cu" "*.Mask") (remove_unused_layers no) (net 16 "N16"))
  (pad "13" thru_hole circle (at 7.625 5.08 180) (size 1.7 1.7) (drill 1) (layers "*.Cu" "*.Mask") (remove_unused_layers no) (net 3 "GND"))
  (pad "14" thru_hole circle (at 7.625 7.62 180) (size 1.7 1.7) (drill 1) (layers "*.Cu" "*.Mask") (remove_unused_layers no) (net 10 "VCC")))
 (gr_rect (start 107.94 78.46) (end 177.94 148.46) (stroke (width 0.05) (type default)) (fill none) (layer "Edge.Cuts"))
 (segment (start 146.04 81.5) (end 146.04 89.08) (width 0.2) (layer "B.Cu") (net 12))
 (segment (start 146.04 89.08) (end 150.03 93.07) (width 0.2) (layer "B.Cu") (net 12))
 (segment (start 124.049899 111.37) (end 119.109899 116.31) (width 0.2) (layer "F.Cu") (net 3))
 (segment (start 117.950101 136.31) (end 119.19 136.31) (width 0.2) (layer "F.Cu") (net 3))
 (segment (start 117.13 135.489899) (end 117.950101 136.31) (width 0.2) (layer "F.Cu") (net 3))
 (segment (start 144.8 112.37) (end 144.53 112.1) (width 0.2) (layer "F.Cu") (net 3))
 (segment (start 125.15 112.1) (end 124.88 112.37) (width 0.2) (layer "F.Cu") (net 3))
 (segment (start 124.88 112.37) (end 124.88 125.934415) (width 0.2) (layer "F.Cu") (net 3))
 (segment (start 131.506346 99.95) (end 158.34 99.95) (width 0.2) (layer "F.Cu") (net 3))
 (segment (start 117.13 133.684415) (end 117.13 135.489899) (width 0.2) (layer "F.Cu") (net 3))
 (segment (start 119.19 136.31) (end 123.13 132.37) (width 0.2) (layer "F.Cu") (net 3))
 (segment (start 119.109899 116.31) (end 117.950101 116.31) (width 0.2) (layer "F.Cu") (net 3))
 (segment (start 123.13 132.37) (end 124.88 132.37) (width 0.2) (layer "F.Cu") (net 3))
 (segment (start 117.950101 116.31) (end 117.13 115.489899) (width 0.2) (layer "F.Cu") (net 3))
 (segment (start 164.8 112.37) (end 163.700001 111.270001) (width 0.2) (layer "F.Cu") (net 3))
 (segment (start 124.88 125.934415) (end 117.13 133.684415) (width 0.2) (layer "F.Cu") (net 3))
 (segment (start 117.13 114.326346) (end 131.506346 99.95) (width 0.2) (layer "F.Cu") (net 3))
 (segment (start 117.13 115.489899) (end 117.13 114.326346) (width 0.2) (layer "F.Cu") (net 3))
 (segment (start 144.53 112.1) (end 125.15 112.1) (width 0.2) (layer "F.Cu") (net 3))
 (segment (start 143.8 111.37) (end 124.049899 111.37) (width 0.2) (layer "F.Cu") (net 3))
 (segment (start 144.8 112.37) (end 143.8 111.37) (width 0.2) (layer "F.Cu") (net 3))
 (segment (start 110.54 102.988478) (end 110.54 101.25) (width 0.2) (layer "B.Cu") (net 3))
 (segment (start 124.88 112.37) (end 119.921522 112.37) (width 0.2) (layer "B.Cu") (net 3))
 (segment (start 160.04 107.61) (end 164.8 112.37) (width 0.2) (layer "B.Cu") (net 3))
 (segment (start 164.88 132.37) (end 164.88 112.45) (width 0.2) (layer "B.Cu") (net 3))
 (segment (start 145.584365 80.2) (end 149.62 80.2) (width 0.2) (layer "B.Cu") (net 3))
 (segment (start 124.88 132.37) (end 144.88 132.37) (width 0.2) (layer "B.Cu") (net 3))
 (segment (start 110.54 101.25) (end 111.84 99.95) (width 0.2) (layer "B.Cu") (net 3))
 (segment (start 164.88 112.45) (end 164.8 112.37) (width 0.2) (layer "B.Cu") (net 3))
 (segment (start 134.78 85.45) (end 138.42 81.81) (width 0.2) (layer "B.Cu") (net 3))
 (segment (start 149.62 80.2) (end 160.04 90.62) (width 0.2) (layer "B.Cu") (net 3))
 (segment (start 138.42 81.81) (end 138.42 81.5) (width 0.2) (layer "B.Cu") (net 3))
 (segment (start 144.94 87.82) (end 144.94 80.844365) (width 0.2) (layer "B.Cu") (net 3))
 (segment (start 138.62 81.5) (end 144.94 87.82) (width 0.2) (layer "B.Cu") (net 3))
 (segment (start 144.94 80.844365) (end 145.584365 80.2) (width 0.2) (layer "B.Cu") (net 3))
 (segment (start 119.921522 112.37) (end 110.54 102.988478) (width 0.2) (layer "B.Cu") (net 3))
 (segment (start 138.42 81.5) (end 138.62 81.5) (width 0.2) (layer "B.Cu") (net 3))
 (segment (start 160.04 90.62) (end 160.04 107.61) (width 0.2) (layer "B.Cu") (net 3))
 (segment (start 144.88 132.37) (end 164.88 132.37) (width 0.2) (layer "B.Cu") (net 3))
 (segment (start 134.303654 96.76) (end 148.88 96.76) (width 0.2) (layer "F.Cu") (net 11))
 (segment (start 133.63 96.086346) (end 134.303654 96.76) (width 0.2) (layer "F.Cu") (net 11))
 (segment (start 143.5 86.216346) (end 135.256346 94.46) (width 0.2) (layer "F.Cu") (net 11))
 (segment (start 134.303654 94.46) (end 133.63 95.133654) (width 0.2) (layer "F.Cu") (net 11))
 (segment (start 148.88 96.76) (end 150.03 95.61) (width 0.2) (layer "F.Cu") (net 11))
 (segment (start 133.63 95.133654) (end 133.63 96.086346) (width 0.2) (layer "F.Cu") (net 11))
 (segment (start 135.256346 94.46) (end 134.303654 94.46) (width 0.2) (layer "F.Cu") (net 11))
 (segment (start 143.5 81.5) (end 143.5 86.216346) (width 0.2) (layer "F.Cu") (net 11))
 (segment (start 139.55 82.91) (end 140.96 81.5) (width 0.2) (layer "F.Cu") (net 10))
 (segment (start 134.78 82.91) (end 139.55 82.91) (width 0.2) (layer "F.Cu") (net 10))
 (segment (start 159.64 102.988478) (end 151.658478 110.97) (width 0.2) (layer "F.Cu") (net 7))
 (segment (start 122.47 110.97) (end 118.53 114.91) (width 0.2) (layer "F.Cu") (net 7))
 (segment (start 151.658478 110.97) (end 122.47 110.97) (width 0.2) (layer "F.Cu") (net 7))
 (segment (start 159.64 92.52) (end 159.64 102.988478) (width 0.2) (layer "F.Cu") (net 7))
 (segment (start 150.03 82.91) (end 159.64 92.52) (width 0.2) (layer "F.Cu") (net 7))
 (segment (start 149.28 94.22) (end 146.5 97) (width 0.2) (layer "B.Cu") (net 14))
 (segment (start 150.506346 94.22) (end 149.28 94.22) (width 0.2) (layer "B.Cu") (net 14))
 (segment (start 133.63 110.09) (end 138.45 114.91) (width 0.2) (layer "B.Cu") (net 14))
 (segment (start 134.303654 97) (end 133.63 97.673654) (width 0.2) (layer "B.Cu") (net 14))
 (segment (start 151.18 86.6) (end 151.18 93.546346) (width 0.2) (layer "B.Cu") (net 14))
 (segment (start 151.18 93.546346) (end 150.506346 94.22) (width 0.2) (layer "B.Cu") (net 14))
 (segment (start 133.63 97.673654) (end 133.63 110.09) (width 0.2) (layer "B.Cu") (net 14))
 (segment (start 146.5 97) (end 134.303654 97) (width 0.2) (layer "B.Cu") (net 14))
 (segment (start 150.03 85.45) (end 151.18 86.6) (width 0.2) (layer "B.Cu") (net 14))
 (segment (start 149.553654 84.3) (end 150.506346 84.3) (width 0.2) (layer "B.Cu") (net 6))
 (segment (start 159.64 93.433654) (end 159.64 113.72) (width 0.2) (layer "B.Cu") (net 6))
 (segment (start 159.64 113.72) (end 158.45 114.91) (width 0.2) (layer "B.Cu") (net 6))
 (segment (start 148.88 84.973654) (end 149.553654 84.3) (width 0.2) (layer "B.Cu") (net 6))
 (segment (start 150.03 87.99) (end 148.88 86.84) (width 0.2) (layer "B.Cu") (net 6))
 (segment (start 150.506346 84.3) (end 159.64 93.433654) (width 0.2) (layer "B.Cu") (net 6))
 (segment (start 148.88 86.84) (end 148.88 84.973654) (width 0.2) (layer "B.Cu") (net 6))
 (segment (start 148.88 89.38) (end 148.88 81.76) (width 0.2) (layer "F.Cu") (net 5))
 (segment (start 138.880101 112.5) (end 118.53 132.850101) (width 0.2) (layer "F.Cu") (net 5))
 (segment (start 160.04 103.154164) (end 149.424164 113.77) (width 0.2) (layer "F.Cu") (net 5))
 (segment (start 148.88 81.76) (end 151.18 81.76) (width 0.2) (layer "F.Cu") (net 5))
 (segment (start 118.53 132.850101) (end 118.53 134.91) (width 0.2) (layer "F.Cu") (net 5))
 (segment (start 144.220101 113.77) (end 142.950101 112.5) (width 0.2) (layer "F.Cu") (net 5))
 (segment (start 142.950101 112.5) (end 138.880101 112.5) (width 0.2) (layer "F.Cu") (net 5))
 (segment (start 151.18 81.76) (end 160.04 90.62) (width 0.2) (layer "F.Cu") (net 5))
 (segment (start 150.03 90.53) (end 148.88 89.38) (width 0.2) (layer "F.Cu") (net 5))
 (segment (start 149.424164 113.77) (end 144.220101 113.77) (width 0.2) (layer "F.Cu") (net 5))
 (segment (start 160.04 90.62) (end 160.04 103.154164) (width 0.2) (layer "F.Cu") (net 5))
 (segment (start 132.2 95.65) (end 118.64 95.65) (width 0.2) (layer "B.Cu") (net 2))
 (segment (start 134.78 93.07) (end 132.2 95.65) (width 0.2) (layer "B.Cu") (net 2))
 (segment (start 118.64 95.65) (end 111.84 102.45) (width 0.2) (layer "B.Cu") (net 2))
 (segment (start 134.78 90.53) (end 119.96 90.53) (width 0.2) (layer "B.Cu") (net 1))
 (segment (start 119.96 90.53) (end 113.04 97.45) (width 0.2) (layer "B.Cu") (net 1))
 (segment (start 113.04 97.45) (end 111.84 97.45) (width 0.2) (layer "B.Cu") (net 1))
 (segment (start 135.93 94.46) (end 155.35 94.46) (width 0.2) (layer "F.Cu") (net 8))
 (segment (start 155.35 94.46) (end 158.34 97.45) (width 0.2) (layer "F.Cu") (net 8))
 (segment (start 134.78 95.61) (end 135.93 94.46) (width 0.2) (layer "F.Cu") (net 8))
 (segment (start 139.08 102.45) (end 158.34 102.45) (width 0.2) (layer "B.Cu") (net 9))
 (segment (start 134.78 98.15) (end 139.08 102.45) (width 0.2) (layer "B.Cu") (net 9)))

